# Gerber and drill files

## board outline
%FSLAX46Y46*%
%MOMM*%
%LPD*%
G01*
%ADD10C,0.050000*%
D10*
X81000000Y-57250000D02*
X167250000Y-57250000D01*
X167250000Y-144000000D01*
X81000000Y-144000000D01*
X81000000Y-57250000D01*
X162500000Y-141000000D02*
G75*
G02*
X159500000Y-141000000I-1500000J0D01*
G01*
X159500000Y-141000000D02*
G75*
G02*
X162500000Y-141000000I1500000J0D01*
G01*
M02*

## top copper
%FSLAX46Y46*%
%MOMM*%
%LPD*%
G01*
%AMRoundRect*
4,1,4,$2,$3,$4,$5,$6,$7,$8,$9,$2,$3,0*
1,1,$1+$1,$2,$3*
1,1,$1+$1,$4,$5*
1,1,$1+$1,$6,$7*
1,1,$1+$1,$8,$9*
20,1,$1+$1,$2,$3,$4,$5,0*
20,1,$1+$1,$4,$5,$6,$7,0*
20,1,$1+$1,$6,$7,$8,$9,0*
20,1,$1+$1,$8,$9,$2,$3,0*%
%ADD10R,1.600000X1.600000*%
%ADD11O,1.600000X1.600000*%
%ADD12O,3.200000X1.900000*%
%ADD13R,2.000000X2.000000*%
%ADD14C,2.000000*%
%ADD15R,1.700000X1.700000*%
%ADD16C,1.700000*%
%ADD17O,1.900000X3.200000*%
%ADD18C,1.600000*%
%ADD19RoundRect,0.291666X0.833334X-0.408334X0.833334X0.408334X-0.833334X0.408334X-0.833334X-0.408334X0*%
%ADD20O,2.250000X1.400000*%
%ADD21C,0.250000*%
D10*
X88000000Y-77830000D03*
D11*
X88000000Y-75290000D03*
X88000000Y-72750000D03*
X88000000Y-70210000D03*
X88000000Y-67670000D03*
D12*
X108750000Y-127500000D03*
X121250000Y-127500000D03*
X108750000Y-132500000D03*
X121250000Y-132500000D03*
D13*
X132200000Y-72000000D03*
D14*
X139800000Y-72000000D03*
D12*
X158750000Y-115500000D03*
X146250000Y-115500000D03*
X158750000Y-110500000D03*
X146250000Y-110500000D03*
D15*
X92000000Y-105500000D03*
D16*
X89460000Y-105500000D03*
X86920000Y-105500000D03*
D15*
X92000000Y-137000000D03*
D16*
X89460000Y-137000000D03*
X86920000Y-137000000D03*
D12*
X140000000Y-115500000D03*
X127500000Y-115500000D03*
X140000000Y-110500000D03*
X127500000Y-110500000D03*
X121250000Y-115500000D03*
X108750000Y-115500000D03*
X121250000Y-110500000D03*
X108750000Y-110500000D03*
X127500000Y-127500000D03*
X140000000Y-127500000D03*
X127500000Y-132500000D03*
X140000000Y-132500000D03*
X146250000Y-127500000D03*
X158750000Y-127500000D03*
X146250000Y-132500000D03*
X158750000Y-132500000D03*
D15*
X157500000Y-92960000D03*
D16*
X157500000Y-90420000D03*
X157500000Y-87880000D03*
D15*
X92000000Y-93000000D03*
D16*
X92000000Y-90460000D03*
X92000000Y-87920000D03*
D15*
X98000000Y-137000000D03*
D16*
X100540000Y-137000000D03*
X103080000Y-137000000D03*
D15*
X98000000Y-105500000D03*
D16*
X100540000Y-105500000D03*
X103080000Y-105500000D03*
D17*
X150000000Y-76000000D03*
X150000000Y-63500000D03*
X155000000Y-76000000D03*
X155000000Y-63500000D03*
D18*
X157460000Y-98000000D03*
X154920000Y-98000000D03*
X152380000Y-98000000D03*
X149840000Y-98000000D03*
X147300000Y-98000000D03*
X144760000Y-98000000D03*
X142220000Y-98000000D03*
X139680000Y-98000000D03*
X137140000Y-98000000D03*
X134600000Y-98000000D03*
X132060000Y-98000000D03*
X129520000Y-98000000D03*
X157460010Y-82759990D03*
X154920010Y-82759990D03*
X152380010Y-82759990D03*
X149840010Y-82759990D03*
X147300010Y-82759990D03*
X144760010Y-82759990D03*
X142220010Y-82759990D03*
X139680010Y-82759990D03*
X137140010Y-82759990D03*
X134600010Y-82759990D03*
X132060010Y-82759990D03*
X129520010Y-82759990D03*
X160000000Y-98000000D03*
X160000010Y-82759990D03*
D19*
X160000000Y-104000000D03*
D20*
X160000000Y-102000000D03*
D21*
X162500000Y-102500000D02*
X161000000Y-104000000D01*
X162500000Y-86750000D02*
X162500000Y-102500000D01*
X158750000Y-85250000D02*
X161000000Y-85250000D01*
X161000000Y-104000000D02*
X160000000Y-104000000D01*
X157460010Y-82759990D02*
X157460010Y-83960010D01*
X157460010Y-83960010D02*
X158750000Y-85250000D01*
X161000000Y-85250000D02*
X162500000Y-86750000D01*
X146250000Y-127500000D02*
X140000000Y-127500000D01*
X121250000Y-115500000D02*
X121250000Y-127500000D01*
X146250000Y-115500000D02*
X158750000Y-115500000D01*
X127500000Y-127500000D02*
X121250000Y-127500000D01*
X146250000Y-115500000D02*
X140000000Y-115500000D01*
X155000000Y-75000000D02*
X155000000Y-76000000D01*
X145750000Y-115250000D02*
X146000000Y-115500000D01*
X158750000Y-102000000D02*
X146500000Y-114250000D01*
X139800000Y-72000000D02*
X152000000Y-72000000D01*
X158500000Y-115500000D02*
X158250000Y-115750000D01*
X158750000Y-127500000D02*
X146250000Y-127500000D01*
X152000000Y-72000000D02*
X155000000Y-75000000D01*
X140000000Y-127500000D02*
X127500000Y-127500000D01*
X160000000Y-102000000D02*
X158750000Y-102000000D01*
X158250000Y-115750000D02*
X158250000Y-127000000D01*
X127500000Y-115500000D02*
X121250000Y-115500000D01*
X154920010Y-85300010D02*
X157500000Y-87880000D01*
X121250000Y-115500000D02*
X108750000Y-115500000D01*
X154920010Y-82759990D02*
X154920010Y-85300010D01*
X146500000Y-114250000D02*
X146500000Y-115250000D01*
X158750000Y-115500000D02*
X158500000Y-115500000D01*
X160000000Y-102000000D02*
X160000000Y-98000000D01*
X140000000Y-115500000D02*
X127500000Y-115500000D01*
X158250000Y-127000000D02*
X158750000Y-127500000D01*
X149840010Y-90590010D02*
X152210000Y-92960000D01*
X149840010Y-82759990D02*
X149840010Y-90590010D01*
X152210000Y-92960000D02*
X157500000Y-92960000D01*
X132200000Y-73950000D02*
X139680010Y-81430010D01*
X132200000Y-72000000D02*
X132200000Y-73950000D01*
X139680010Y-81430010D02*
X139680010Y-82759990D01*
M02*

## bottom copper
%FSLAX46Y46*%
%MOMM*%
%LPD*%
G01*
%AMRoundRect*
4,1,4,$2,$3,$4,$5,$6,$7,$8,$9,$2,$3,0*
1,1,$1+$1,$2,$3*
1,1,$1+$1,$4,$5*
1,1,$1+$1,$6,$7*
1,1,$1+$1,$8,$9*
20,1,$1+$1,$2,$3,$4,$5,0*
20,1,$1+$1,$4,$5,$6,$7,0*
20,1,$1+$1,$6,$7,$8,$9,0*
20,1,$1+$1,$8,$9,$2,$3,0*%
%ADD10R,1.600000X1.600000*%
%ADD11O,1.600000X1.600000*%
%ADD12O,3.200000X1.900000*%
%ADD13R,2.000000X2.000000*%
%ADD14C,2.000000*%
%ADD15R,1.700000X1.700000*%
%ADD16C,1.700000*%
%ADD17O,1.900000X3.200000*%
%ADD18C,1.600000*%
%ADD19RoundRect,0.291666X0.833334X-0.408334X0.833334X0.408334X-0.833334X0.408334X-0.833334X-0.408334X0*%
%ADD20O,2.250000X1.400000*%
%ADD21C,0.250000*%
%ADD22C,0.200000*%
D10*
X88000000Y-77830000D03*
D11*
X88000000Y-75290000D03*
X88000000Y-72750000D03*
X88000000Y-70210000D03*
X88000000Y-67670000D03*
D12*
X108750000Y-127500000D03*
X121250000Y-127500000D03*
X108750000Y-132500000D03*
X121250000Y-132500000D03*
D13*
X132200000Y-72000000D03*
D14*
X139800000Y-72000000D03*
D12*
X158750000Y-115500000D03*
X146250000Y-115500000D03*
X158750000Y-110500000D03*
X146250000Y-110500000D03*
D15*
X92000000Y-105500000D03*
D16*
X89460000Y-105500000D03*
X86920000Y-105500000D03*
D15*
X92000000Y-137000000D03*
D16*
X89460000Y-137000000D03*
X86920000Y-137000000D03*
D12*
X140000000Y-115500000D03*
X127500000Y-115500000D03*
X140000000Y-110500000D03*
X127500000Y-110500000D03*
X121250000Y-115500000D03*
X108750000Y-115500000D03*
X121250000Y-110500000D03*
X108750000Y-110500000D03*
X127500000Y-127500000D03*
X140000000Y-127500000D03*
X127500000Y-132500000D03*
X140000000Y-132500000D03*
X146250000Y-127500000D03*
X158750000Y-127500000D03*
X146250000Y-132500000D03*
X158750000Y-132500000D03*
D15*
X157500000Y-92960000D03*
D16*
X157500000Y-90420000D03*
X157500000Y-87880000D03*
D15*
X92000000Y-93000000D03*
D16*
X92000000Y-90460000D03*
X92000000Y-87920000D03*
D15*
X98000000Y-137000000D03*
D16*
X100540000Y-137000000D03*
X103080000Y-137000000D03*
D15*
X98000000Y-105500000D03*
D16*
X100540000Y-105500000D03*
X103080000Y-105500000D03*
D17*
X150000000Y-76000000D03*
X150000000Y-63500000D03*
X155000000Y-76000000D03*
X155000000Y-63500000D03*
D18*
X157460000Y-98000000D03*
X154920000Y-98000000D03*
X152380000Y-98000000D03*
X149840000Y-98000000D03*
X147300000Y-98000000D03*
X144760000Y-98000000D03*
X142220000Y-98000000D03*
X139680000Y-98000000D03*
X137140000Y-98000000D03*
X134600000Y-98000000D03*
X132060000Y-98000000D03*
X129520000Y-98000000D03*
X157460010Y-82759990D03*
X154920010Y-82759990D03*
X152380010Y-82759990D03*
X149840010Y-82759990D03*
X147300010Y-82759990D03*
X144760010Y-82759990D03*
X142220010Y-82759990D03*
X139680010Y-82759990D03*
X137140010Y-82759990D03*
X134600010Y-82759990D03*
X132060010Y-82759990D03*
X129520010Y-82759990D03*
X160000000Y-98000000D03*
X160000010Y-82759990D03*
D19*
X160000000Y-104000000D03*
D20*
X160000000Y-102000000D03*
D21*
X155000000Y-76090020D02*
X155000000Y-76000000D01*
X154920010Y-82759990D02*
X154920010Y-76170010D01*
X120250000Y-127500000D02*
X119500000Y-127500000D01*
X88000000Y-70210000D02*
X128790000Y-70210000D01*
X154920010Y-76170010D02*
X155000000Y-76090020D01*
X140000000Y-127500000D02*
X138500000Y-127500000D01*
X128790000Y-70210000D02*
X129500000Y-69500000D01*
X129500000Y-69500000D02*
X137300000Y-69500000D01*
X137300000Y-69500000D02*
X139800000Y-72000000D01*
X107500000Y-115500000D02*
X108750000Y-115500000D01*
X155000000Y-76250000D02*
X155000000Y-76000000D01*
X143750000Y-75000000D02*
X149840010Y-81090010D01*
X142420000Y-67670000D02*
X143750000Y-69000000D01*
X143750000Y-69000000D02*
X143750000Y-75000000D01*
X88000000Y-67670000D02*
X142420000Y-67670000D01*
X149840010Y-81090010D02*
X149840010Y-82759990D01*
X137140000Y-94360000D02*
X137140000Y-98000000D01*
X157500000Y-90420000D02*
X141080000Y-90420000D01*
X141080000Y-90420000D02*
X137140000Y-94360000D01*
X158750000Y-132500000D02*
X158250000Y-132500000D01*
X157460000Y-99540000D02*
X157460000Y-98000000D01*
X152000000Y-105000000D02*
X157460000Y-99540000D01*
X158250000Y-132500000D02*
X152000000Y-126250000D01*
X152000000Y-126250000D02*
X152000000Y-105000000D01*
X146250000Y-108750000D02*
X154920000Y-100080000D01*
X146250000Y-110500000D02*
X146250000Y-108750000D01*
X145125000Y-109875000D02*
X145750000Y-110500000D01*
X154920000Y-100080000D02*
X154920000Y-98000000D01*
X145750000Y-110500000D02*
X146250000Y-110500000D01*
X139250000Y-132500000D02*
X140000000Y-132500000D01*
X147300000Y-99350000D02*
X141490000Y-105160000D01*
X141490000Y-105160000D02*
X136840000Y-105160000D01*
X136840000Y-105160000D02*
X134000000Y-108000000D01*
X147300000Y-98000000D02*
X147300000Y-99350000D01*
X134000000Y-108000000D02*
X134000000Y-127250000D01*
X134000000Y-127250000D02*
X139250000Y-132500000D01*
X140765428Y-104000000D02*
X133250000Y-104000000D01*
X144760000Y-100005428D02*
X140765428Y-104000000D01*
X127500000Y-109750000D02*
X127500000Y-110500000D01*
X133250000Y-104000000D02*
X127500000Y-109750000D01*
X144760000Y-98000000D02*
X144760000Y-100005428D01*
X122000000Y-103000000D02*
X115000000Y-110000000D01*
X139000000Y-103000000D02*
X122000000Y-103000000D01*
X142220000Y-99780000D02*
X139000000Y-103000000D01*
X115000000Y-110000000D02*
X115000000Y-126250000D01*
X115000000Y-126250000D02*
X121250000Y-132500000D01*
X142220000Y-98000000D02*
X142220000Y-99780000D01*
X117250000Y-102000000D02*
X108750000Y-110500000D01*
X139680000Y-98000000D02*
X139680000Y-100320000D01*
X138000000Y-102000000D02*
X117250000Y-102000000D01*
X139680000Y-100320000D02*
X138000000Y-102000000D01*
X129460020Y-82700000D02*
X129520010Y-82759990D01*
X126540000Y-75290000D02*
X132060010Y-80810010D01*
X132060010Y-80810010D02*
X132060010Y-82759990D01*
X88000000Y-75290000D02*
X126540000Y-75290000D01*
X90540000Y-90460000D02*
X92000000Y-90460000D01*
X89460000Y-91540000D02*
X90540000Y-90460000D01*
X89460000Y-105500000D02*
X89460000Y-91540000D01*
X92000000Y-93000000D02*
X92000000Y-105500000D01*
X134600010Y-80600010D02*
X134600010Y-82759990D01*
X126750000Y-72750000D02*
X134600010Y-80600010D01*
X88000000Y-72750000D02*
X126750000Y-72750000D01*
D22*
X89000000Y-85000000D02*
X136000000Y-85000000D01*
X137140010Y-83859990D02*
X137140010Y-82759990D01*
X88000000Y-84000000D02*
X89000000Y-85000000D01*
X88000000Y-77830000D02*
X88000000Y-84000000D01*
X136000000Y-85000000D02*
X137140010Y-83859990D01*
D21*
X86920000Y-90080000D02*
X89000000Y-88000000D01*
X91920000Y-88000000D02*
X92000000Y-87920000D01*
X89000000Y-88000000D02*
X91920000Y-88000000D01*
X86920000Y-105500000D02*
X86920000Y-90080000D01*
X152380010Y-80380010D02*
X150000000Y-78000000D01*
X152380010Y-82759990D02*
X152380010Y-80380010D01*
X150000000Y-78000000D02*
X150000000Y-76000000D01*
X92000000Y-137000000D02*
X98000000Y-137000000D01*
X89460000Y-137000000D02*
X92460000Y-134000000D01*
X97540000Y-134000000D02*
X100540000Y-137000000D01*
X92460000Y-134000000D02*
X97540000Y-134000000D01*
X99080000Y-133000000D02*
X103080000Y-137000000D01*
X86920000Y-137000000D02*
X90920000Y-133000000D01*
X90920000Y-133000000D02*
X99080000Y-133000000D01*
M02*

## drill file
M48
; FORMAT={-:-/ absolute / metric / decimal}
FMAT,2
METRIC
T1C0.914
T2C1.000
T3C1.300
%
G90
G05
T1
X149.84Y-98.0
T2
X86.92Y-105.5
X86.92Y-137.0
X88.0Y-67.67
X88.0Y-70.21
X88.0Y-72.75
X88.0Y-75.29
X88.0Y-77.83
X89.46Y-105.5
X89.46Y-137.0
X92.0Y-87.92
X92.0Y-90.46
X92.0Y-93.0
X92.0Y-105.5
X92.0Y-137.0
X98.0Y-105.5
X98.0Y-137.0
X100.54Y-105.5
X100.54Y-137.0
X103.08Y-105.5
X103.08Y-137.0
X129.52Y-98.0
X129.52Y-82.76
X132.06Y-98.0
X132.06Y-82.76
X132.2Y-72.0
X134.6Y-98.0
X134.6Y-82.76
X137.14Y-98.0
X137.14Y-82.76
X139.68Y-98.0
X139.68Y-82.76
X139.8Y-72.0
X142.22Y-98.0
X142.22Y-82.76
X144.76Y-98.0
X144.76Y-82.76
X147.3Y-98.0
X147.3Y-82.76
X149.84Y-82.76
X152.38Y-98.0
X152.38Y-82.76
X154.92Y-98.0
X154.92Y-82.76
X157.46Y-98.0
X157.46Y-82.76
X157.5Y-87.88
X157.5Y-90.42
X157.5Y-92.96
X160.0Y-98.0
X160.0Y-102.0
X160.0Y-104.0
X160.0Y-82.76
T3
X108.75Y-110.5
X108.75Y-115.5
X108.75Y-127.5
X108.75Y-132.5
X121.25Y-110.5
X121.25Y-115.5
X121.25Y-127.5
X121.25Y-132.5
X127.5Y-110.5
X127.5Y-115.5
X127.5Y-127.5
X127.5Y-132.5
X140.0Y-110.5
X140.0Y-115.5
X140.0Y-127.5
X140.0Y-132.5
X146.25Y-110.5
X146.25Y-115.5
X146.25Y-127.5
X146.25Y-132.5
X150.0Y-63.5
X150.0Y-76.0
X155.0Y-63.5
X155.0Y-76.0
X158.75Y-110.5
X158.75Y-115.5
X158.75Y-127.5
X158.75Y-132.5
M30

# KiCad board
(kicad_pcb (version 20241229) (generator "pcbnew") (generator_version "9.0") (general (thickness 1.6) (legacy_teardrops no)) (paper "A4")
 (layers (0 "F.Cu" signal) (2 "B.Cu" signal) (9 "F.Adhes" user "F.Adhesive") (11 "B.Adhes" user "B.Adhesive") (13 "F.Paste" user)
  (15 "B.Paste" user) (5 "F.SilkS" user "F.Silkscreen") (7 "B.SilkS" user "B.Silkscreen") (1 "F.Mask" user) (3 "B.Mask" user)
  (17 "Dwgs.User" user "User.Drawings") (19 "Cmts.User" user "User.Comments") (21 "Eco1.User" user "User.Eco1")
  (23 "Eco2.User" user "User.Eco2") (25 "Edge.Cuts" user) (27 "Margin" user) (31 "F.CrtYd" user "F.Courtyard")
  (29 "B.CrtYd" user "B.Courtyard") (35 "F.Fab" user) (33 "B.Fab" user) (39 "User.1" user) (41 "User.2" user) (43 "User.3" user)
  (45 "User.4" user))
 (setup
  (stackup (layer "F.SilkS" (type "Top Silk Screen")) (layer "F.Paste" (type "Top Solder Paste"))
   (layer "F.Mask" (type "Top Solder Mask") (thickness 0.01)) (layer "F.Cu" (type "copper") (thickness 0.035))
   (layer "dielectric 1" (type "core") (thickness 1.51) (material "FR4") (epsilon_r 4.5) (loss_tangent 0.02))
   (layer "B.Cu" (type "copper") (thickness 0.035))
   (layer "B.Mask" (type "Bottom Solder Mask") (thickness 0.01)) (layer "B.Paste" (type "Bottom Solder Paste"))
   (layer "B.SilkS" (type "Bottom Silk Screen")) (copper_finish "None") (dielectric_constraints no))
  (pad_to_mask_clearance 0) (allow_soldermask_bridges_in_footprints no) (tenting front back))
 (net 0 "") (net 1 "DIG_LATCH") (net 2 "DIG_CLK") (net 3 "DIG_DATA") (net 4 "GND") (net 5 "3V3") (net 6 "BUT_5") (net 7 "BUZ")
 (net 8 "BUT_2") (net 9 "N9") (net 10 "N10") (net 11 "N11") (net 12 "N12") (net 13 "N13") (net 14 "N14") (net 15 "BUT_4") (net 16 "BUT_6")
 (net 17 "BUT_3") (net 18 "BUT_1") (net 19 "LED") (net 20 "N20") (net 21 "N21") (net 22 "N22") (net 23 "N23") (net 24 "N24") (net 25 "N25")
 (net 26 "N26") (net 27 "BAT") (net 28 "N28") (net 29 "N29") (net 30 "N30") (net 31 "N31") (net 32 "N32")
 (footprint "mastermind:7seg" (layer "F.Cu") (at 94.5 69.25)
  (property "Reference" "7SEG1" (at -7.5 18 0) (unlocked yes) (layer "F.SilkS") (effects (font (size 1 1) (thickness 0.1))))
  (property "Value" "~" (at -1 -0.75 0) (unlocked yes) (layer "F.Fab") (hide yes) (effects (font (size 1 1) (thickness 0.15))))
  (pad "1" thru_hole rect (at -6.5 8.58 180) (size 1.6 1.6) (drill 1) (layers "*.Cu" "*.Mask") (remove_unused_layers no) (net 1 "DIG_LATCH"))
  (pad "2" thru_hole oval (at -6.5 6.04 180) (size 1.6 1.6) (drill 1) (layers "*.Cu" "*.Mask") (remove_unused_layers no) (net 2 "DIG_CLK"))
  (pad "3" thru_hole oval (at -6.5 3.5 180) (size 1.6 1.6) (drill 1) (layers "*.Cu" "*.Mask") (remove_unused_layers no) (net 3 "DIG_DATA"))
  (pad "4" thru_hole oval (at -6.5 0.96 180) (size 1.6 1.6) (drill 1) (layers "*.Cu" "*.Mask") (remove_unused_layers no) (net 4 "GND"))
  (pad "5" thru_hole oval (at -6.5 -1.58 180) (size 1.6 1.6) (drill 1) (layers "*.Cu" "*.Mask") (remove_unused_layers no) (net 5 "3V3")))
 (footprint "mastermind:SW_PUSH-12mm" (layer "F.Cu") (at 108.75 127.5)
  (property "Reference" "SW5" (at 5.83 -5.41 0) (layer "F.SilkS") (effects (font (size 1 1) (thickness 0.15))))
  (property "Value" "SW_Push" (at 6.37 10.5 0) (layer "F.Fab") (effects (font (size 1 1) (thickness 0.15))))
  (pad "1" thru_hole oval (at 0 0) (size 3.2 1.9) (drill 1.3) (layers "*.Cu" "*.Mask") (remove_unused_layers no) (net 4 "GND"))
  (pad "1" thru_hole oval (at 12.5 0) (size 3.2 1.9) (drill 1.3) (layers "*.Cu" "*.Mask") (remove_unused_layers no) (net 4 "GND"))
  (pad "2" thru_hole oval (at 0 5) (size 3.2 1.9) (drill 1.3) (layers "*.Cu" "*.Mask") (remove_unused_layers no) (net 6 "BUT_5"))
  (pad "2" thru_hole oval (at 12.5 5) (size 3.2 1.9) (drill 1.3) (layers "*.Cu" "*.Mask") (remove_unused_layers no) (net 6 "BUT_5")))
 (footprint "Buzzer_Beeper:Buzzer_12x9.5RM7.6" (layer "F.Cu") (at 132.2 72)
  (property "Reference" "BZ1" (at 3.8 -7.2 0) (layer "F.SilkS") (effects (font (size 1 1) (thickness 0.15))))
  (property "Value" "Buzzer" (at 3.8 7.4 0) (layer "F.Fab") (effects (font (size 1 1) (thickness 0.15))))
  (pad "1" thru_hole rect (at 0 0) (size 2 2) (drill 1) (layers "*.Cu" "*.Mask") (remove_unused_layers no) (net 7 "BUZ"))
  (pad "2" thru_hole circle (at 7.6 0) (size 2 2) (drill 1) (layers "*.Cu" "*.Mask") (remove_unused_layers no) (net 4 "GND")))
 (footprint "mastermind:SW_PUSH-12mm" (layer "F.Cu") (at 158.75 115.5 180)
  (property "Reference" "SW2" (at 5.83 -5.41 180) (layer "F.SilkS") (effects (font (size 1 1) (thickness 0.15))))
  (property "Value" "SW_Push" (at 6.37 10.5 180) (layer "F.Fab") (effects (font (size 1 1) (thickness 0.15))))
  (pad "1" thru_hole oval (at 0 0 180) (size 3.2 1.9) (drill 1.3) (layers "*.Cu" "*.Mask") (remove_unused_layers no) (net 4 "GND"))
  (pad "1" thru_hole oval (at 12.5 0 180) (size 3.2 1.9) (drill 1.3) (layers "*.Cu" "*.Mask") (remove_unused_layers no) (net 4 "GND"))
  (pad "2" thru_hole oval (at 0 5 180) (size 3.2 1.9) (drill 1.3) (layers "*.Cu" "*.Mask") (remove_unused_layers no) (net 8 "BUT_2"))
  (pad "2" thru_hole oval (at 12.5 5 180) (size 3.2 1.9) (drill 1.3) (layers "*.Cu" "*.Mask") (remove_unused_layers no) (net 8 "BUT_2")))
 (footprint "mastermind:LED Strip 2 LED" (layer "F.Cu") (at 89.75 129.75 -90)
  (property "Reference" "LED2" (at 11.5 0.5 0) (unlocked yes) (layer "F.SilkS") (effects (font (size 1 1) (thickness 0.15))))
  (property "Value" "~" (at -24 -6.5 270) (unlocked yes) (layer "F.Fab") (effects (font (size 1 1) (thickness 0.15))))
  (pad "1" thru_hole rect (at -24.25 -2.25 270) (size 1.7 1.7) (drill 1) (layers "*.Cu" "*.Mask") (remove_unused_layers no) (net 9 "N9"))
  (pad "2" thru_hole circle (at -24.25 0.29 270) (size 1.7 1.7) (drill 1) (layers "*.Cu" "*.Mask") (remove_unused_layers no) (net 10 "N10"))
  (pad "3" thru_hole circle (at -24.25 2.83 270) (size 1.7 1.7) (drill 1) (layers "*.Cu" "*.Mask") (remove_unused_layers no) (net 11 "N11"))
  (pad "4" thru_hole rect (at 7.25 -2.25 270) (size 1.7 1.7) (drill 1) (layers "*.Cu" "*.Mask") (remove_unused_layers no) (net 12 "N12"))
  (pad "5" thru_hole circle (at 7.25 0.29 270) (size 1.7 1.7) (drill 1) (layers "*.Cu" "*.Mask") (remove_unused_layers no) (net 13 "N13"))
  (pad "6" thru_hole circle (at 7.25 2.83 270) (size 1.7 1.7) (drill 1) (layers "*.Cu" "*.Mask") (remove_unused_layers no) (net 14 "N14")))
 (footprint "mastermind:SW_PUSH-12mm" (layer "F.Cu") (at 140 115.5 180)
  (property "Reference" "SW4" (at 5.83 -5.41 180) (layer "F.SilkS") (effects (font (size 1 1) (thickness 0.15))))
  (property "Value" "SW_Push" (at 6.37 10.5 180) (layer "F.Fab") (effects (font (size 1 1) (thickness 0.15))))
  (pad "1" thru_hole oval (at 0 0 180) (size 3.2 1.9) (drill 1.3) (layers "*.Cu" "*.Mask") (remove_unused_layers no) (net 4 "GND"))
  (pad "1" thru_hole oval (at 12.5 0 180) (size 3.2 1.9) (drill 1.3) (layers "*.Cu" "*.Mask") (remove_unused_layers no) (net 4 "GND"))
  (pad "2" thru_hole oval (at 0 5 180) (size 3.2 1.9) (drill 1.3) (layers "*.Cu" "*.Mask") (remove_unused_layers no) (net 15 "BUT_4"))
  (pad "2" thru_hole oval (at 12.5 5 180) (size 3.2 1.9) (drill 1.3) (layers "*.Cu" "*.Mask") (remove_unused_layers no) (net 15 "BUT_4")))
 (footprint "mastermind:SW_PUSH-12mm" (layer "F.Cu") (at 121.25 115.5 180)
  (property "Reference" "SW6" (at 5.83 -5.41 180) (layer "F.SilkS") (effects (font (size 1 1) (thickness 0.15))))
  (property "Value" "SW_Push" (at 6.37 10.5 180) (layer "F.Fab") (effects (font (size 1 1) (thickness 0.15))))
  (pad "1" thru_hole oval (at 0 0 180) (size 3.2 1.9) (drill 1.3) (layers "*.Cu" "*.Mask") (remove_unused_layers no) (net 4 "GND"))
  (pad "1" thru_hole oval (at 12.5 0 180) (size 3.2 1.9) (drill 1.3) (layers "*.Cu" "*.Mask") (remove_unused_layers no) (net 4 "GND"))
  (pad "2" thru_hole oval (at 0 5 180) (size 3.2 1.9) (drill 1.3) (layers "*.Cu" "*.Mask") (remove_unused_layers no) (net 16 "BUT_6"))
  (pad "2" thru_hole oval (at 12.5 5 180) (size 3.2 1.9) (drill 1.3) (layers "*.Cu" "*.Mask") (remove_unused_layers no) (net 16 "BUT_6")))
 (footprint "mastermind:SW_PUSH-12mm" (layer "F.Cu") (at 127.5 127.5)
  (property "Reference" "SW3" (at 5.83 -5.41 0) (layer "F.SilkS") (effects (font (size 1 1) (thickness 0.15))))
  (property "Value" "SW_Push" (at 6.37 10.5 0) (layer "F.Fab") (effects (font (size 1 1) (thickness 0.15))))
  (pad "1" thru_hole oval (at 0 0) (size 3.2 1.9) (drill 1.3) (layers "*.Cu" "*.Mask") (remove_unused_layers no) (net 4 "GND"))
  (pad "1" thru_hole oval (at 12.5 0) (size 3.2 1.9) (drill 1.3) (layers "*.Cu" "*.Mask") (remove_unused_layers no) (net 4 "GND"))
  (pad "2" thru_hole oval (at 0 5) (size 3.2 1.9) (drill 1.3) (layers "*.Cu" "*.Mask") (remove_unused_layers no) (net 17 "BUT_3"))
  (pad "2" thru_hole oval (at 12.5 5) (size 3.2 1.9) (drill 1.3) (layers "*.Cu" "*.Mask") (remove_unused_layers no) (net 17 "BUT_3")))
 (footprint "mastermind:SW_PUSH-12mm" (layer "F.Cu") (at 146.25 127.5)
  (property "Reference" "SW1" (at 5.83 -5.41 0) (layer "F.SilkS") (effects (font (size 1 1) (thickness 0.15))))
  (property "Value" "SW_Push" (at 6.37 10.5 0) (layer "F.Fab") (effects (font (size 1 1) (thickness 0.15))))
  (pad "1" thru_hole oval (at 0 0) (size 3.2 1.9) (drill 1.3) (layers "*.Cu" "*.Mask") (remove_unused_layers no) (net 4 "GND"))
  (pad "1" thru_hole oval (at 12.5 0) (size 3.2 1.9) (drill 1.3) (layers "*.Cu" "*.Mask") (remove_unused_layers no) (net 4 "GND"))
  (pad "2" thru_hole oval (at 0 5) (size 3.2 1.9) (drill 1.3) (layers "*.Cu" "*.Mask") (remove_unused_layers no) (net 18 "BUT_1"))
  (pad "2" thru_hole oval (at 12.5 5) (size 3.2 1.9) (drill 1.3) (layers "*.Cu" "*.Mask") (remove_unused_layers no) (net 18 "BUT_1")))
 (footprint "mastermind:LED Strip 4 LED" (layer "F.Cu") (at 133.25 90.71 180)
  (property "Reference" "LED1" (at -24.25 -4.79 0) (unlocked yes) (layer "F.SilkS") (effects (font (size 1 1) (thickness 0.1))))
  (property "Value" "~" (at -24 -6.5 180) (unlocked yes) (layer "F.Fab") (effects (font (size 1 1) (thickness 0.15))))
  (pad "1" thru_hole rect (at -24.25 -2.25 180) (size 1.7 1.7) (drill 1) (layers "*.Cu" "*.Mask") (remove_unused_layers no) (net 5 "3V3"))
  (pad "2" thru_hole circle (at -24.25 0.29 180) (size 1.7 1.7) (drill 1) (layers "*.Cu" "*.Mask") (remove_unused_layers no) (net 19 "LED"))
  (pad "3" thru_hole circle (at -24.25 2.83 180) (size 1.7 1.7) (drill 1) (layers "*.Cu" "*.Mask") (remove_unused_layers no) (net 4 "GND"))
  (pad "4" thru_hole rect (at 41.25 -2.29 180) (size 1.7 1.7) (drill 1) (layers "*.Cu" "*.Mask") (remove_unused_layers no) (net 9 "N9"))
  (pad "5" thru_hole circle (at 41.25 0.25 180) (size 1.7 1.7) (drill 1) (layers "*.Cu" "*.Mask") (remove_unused_layers no) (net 10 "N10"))
  (pad "6" thru_hole circle (at 41.25 2.79 180) (size 1.7 1.7) (drill 1) (layers "*.Cu" "*.Mask") (remove_unused_layers no) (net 11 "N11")))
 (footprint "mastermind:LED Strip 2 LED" (layer "F.Cu") (at 100.25 112.75 90)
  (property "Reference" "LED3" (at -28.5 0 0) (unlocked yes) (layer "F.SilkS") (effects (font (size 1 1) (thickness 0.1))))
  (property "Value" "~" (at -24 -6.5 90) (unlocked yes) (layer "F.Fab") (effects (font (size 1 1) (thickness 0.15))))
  (pad "1" thru_hole rect (at -24.25 -2.25 90) (size 1.7 1.7) (drill 1) (layers "*.Cu" "*.Mask") (remove_unused_layers no) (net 12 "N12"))
  (pad "2" thru_hole circle (at -24.25 0.29 90) (size 1.7 1.7) (drill 1) (layers "*.Cu" "*.Mask") (remove_unused_layers no) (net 13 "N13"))
  (pad "3" thru_hole circle (at -24.25 2.83 90) (size 1.7 1.7) (drill 1) (layers "*.Cu" "*.Mask") (remove_unused_layers no) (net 14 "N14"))
  (pad "4" thru_hole rect (at 7.25 -2.25 90) (size 1.7 1.7) (drill 1) (layers "*.Cu" "*.Mask") (remove_unused_layers no) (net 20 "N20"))
  (pad "5" thru_hole circle (at 7.25 0.29 90) (size 1.7 1.7) (drill 1) (layers "*.Cu" "*.Mask") (remove_unused_layers no) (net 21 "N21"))
  (pad "6" thru_hole circle (at 7.25 2.83 90) (size 1.7 1.7) (drill 1) (layers "*.Cu" "*.Mask") (remove_unused_layers no) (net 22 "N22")))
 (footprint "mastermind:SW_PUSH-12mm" (layer "F.Cu") (at 150 76 90)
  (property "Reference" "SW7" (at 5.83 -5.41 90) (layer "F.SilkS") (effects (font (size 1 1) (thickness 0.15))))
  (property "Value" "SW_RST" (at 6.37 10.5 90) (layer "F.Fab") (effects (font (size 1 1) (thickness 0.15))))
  (pad "1" thru_hole oval (at 0 0 90) (size 3.2 1.9) (drill 1.3) (layers "*.Cu" "*.Mask") (remove_unused_layers no) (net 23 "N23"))
  (pad "1" thru_hole oval (at 12.5 0 90) (size 3.2 1.9) (drill 1.3) (layers "*.Cu" "*.Mask") (remove_unused_layers no) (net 23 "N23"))
  (pad "2" thru_hole oval (at 0 5 90) (size 3.2 1.9) (drill 1.3) (layers "*.Cu" "*.Mask") (remove_unused_layers no) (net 4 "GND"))
  (pad "2" thru_hole oval (at 12.5 5 90) (size 3.2 1.9) (drill 1.3) (layers "*.Cu" "*.Mask") (remove_unused_layers no) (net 4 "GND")))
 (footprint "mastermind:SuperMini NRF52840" (layer "B.Cu") (at 160 98 90)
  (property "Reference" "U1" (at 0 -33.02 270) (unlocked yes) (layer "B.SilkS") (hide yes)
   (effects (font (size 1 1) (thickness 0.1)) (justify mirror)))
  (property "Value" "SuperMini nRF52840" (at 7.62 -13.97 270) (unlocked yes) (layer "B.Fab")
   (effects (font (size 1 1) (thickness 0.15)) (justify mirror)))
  (pad "1" thru_hole circle (at 0 -2.54 180) (size 1.6 1.6) (drill 1) (layers "*.Cu" "*.Mask") (remove_unused_layers no) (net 18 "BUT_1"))
  (pad "2" thru_hole circle (at 0 -5.08 180) (size 1.6 1.6) (drill 1) (layers "*.Cu" "*.Mask") (remove_unused_layers no) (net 8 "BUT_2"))
  (pad "3" thru_hole circle (at 0 -7.62 180) (size 1.6 1.6) (drill 1) (layers "*.Cu" "*.Mask") (remove_unused_layers no) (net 4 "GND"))
  (pad "4" thru_hole circle (at 0 -10.16) (size 1.6 1.6) (drill 0.9144) (layers "*.Cu" "*.Mask") (remove_unused_layers no) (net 4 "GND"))
  (pad "5" thru_hole circle (at 0 -12.7 180) (size 1.6 1.6) (drill 1) (layers "*.Cu" "*.Mask") (remove_unused_layers no) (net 17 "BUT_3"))
  (pad "6" thru_hole circle (at 0 -15.24 180) (size 1.6 1.6) (drill 1) (layers "*.Cu" "*.Mask") (remove_unused_layers no) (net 15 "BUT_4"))
  (pad "7" thru_hole circle (at 0 -17.78 180) (size 1.6 1.6) (drill 1) (layers "*.Cu" "*.Mask") (remove_unused_layers no) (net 6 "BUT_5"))
  (pad "8" thru_hole circle (at 0 -20.32 180) (size 1.6 1.6) (drill 1) (layers "*.Cu" "*.Mask") (remove_unused_layers no) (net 16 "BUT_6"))
  (pad "9" thru_hole circle (at 0 -22.86 180) (size 1.6 1.6) (drill 1) (layers "*.Cu" "*.Mask") (remove_unused_layers no) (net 19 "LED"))
  (pad "10" thru_hole circle (at 0 -25.4 180) (size 1.6 1.6) (drill 1) (layers "*.Cu" "*.Mask") (remove_unused_layers no) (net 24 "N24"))
  (pad "11" thru_hole circle (at 0 -27.94 180) (size 1.6 1.6) (drill 1) (layers "*.Cu" "*.Mask") (remove_unused_layers no) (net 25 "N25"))
  (pad "12" thru_hole circle (at 0 -30.48 180) (size 1.6 1.6) (drill 1) (layers "*.Cu" "*.Mask") (remove_unused_layers no) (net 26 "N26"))
  (pad "13" thru_hole circle (at 15.24001 -2.53999) (size 1.6 1.6) (drill 1) (layers "*.Cu" "*.Mask") (remove_unused_layers no)
   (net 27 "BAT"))
  (pad "14" thru_hole circle (at 15.24001 -5.07999) (size 1.6 1.6) (drill 1) (layers "*.Cu" "*.Mask") (remove_unused_layers no)
   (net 4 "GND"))
  (pad "15" thru_hole circle (at 15.24001 -7.61999) (size 1.6 1.6) (drill 1) (layers "*.Cu" "*.Mask") (remove_unused_layers no)
   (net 23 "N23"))
  (pad "16" thru_hole circle (at 15.24001 -10.15999) (size 1.6 1.6) (drill 1) (layers "*.Cu" "*.Mask") (remove_unused_layers no)
   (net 5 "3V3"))
  (pad "17" thru_hole circle (at 15.24001 -12.69999) (size 1.6 1.6) (drill 1) (layers "*.Cu" "*.Mask") (remove_unused_layers no)
   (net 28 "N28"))
  (pad "18" thru_hole circle (at 15.24001 -15.23999) (size 1.6 1.6) (drill 1) (layers "*.Cu" "*.Mask") (remove_unused_layers no)
   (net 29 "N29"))
  (pad "19" thru_hole circle (at 15.24001 -17.77999) (size 1.6 1.6) (drill 1) (layers "*.Cu" "*.Mask") (remove_unused_layers no)
   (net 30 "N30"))
  (pad "20" thru_hole circle (at 15.24001 -20.31999) (size 1.6 1.6) (drill 1) (layers "*.Cu" "*.Mask") (remove_unused_layers no)
   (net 7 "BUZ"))
  (pad "21" thru_hole circle (at 15.24001 -22.85999) (size 1.6 1.6) (drill 1) (layers "*.Cu" "*.Mask") (remove_unused_layers no)
   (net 1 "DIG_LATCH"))
  (pad "22" thru_hole circle (at 15.24001 -25.39999) (size 1.6 1.6) (drill 1) (layers "*.Cu" "*.Mask") (remove_unused_layers no)
   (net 3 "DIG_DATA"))
  (pad "23" thru_hole circle (at 15.24001 -27.93999) (size 1.6 1.6) (drill 1) (layers "*.Cu" "*.Mask") (remove_unused_layers no)
   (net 2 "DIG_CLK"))
  (pad "24" thru_hole circle (at 15.24001 -30.47999 180) (size 1.6 1.6) (drill 1) (layers "*.Cu" "*.Mask") (remove_unused_layers no)
   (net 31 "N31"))
  (pad "28" thru_hole circle (at 0 0 180) (size 1.6 1.6) (drill 1) (layers "*.Cu" "*.Mask") (remove_unused_layers no) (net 4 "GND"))
  (pad "29" thru_hole circle (at 15.24001 0.00001) (size 1.6 1.6) (drill 1) (layers "*.Cu" "*.Mask") (remove_unused_layers no)
   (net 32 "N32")))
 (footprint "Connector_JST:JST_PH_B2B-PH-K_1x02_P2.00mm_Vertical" (layer "B.Cu") (at 160 104 90)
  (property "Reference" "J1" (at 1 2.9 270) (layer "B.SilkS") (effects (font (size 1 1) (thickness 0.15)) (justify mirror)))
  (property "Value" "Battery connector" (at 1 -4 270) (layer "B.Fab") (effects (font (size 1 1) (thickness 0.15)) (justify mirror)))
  (pad "1" thru_hole roundrect (at 0 0 90) (size 1.4 2.25) (drill 1) (layers "*.Cu" "*.Mask") (remove_unused_layers no)
   (roundrect_rratio 0.208333) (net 27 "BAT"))
  (pad "2" thru_hole oval (at 2 0 90) (size 1.4 2.25) (drill 1) (layers "*.Cu" "*.Mask") (remove_unused_layers no) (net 4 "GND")))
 (gr_rect (start 81 57.25) (end 167.25 144) (stroke (width 0.05) (type default)) (fill no) (layer "Edge.Cuts"))
 (gr_circle (center 161 141) (end 162.5 141) (stroke (width 0.05) (type solid)) (fill no) (layer "Edge.Cuts"))
 (segment (start 162.5 102.5) (end 161 104) (width 0.25) (layer "F.Cu") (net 27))
 (segment (start 162.5 86.75) (end 162.5 102.5) (width 0.25) (layer "F.Cu") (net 27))
 (segment (start 158.75 85.25) (end 161 85.25) (width 0.25) (layer "F.Cu") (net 27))
 (segment (start 161 104) (end 160 104) (width 0.25) (layer "F.Cu") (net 27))
 (segment (start 157.46001 82.75999) (end 157.46001 83.96001) (width 0.25) (layer "F.Cu") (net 27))
 (segment (start 157.46001 83.96001) (end 158.75 85.25) (width 0.25) (layer "F.Cu") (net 27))
 (segment (start 161 85.25) (end 162.5 86.75) (width 0.25) (layer "F.Cu") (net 27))
 (segment (start 146.25 127.5) (end 140 127.5) (width 0.25) (layer "F.Cu") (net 4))
 (segment (start 121.25 115.5) (end 121.25 127.5) (width 0.25) (layer "F.Cu") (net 4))
 (segment (start 146.25 115.5) (end 158.75 115.5) (width 0.25) (layer "F.Cu") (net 4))
 (segment (start 127.5 127.5) (end 121.25 127.5) (width 0.25) (layer "F.Cu") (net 4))
 (segment (start 146.25 115.5) (end 140 115.5) (width 0.25) (layer "F.Cu") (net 4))
 (segment (start 155 75) (end 155 76) (width 0.25) (layer "F.Cu") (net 4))
 (segment (start 145.75 115.25) (end 146 115.5) (width 0.25) (layer "F.Cu") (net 4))
 (segment (start 158.75 102) (end 146.5 114.25) (width 0.25) (layer "F.Cu") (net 4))
 (segment (start 139.8 72) (end 152 72) (width 0.25) (layer "F.Cu") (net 4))
 (segment (start 158.5 115.5) (end 158.25 115.75) (width 0.25) (layer "F.Cu") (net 4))
 (segment (start 158.75 127.5) (end 146.25 127.5) (width 0.25) (layer "F.Cu") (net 4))
 (segment (start 152 72) (end 155 75) (width 0.25) (layer "F.Cu") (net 4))
 (segment (start 140 127.5) (end 127.5 127.5) (width 0.25) (layer "F.Cu") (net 4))
 (segment (start 160 102) (end 158.75 102) (width 0.25) (layer "F.Cu") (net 4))
 (segment (start 158.25 115.75) (end 158.25 127) (width 0.25) (layer "F.Cu") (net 4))
 (segment (start 127.5 115.5) (end 121.25 115.5) (width 0.25) (layer "F.Cu") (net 4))
 (segment (start 154.92001 85.30001) (end 157.5 87.88) (width 0.25) (layer "F.Cu") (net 4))
 (segment (start 121.25 115.5) (end 108.75 115.5) (width 0.25) (layer "F.Cu") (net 4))
 (segment (start 154.92001 82.75999) (end 154.92001 85.30001) (width 0.25) (layer "F.Cu") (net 4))
 (segment (start 146.5 114.25) (end 146.5 115.25) (width 0.25) (layer "F.Cu") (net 4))
 (segment (start 158.75 115.5) (end 158.5 115.5) (width 0.25) (layer "F.Cu") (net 4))
 (segment (start 160 102) (end 160 98) (width 0.25) (layer "F.Cu") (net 4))
 (segment (start 140 115.5) (end 127.5 115.5) (width 0.25) (layer "F.Cu") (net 4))
 (segment (start 158.25 127) (end 158.75 127.5) (width 0.25) (layer "F.Cu") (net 4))
 (segment (start 155 76.09002) (end 155 76) (width 0.25) (layer "B.Cu") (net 4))
 (segment (start 154.92001 82.75999) (end 154.92001 76.17001) (width 0.25) (layer "B.Cu") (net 4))
 (segment (start 120.25 127.5) (end 119.5 127.5) (width 0.25) (layer "B.Cu") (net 4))
 (segment (start 88 70.21) (end 128.79 70.21) (width 0.25) (layer "B.Cu") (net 4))
 (segment (start 154.92001 76.17001) (end 155 76.09002) (width 0.25) (layer "B.Cu") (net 4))
 (segment (start 140 127.5) (end 138.5 127.5) (width 0.25) (layer "B.Cu") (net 4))
 (segment (start 128.79 70.21) (end 129.5 69.5) (width 0.25) (layer "B.Cu") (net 4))
 (segment (start 129.5 69.5) (end 137.3 69.5) (width 0.25) (layer "B.Cu") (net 4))
 (segment (start 137.3 69.5) (end 139.8 72) (width 0.25) (layer "B.Cu") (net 4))
 (segment (start 107.5 115.5) (end 108.75 115.5) (width 0.25) (layer "B.Cu") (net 4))
 (segment (start 155 76.25) (end 155 76) (width 0.25) (layer "B.Cu") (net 4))
 (segment (start 149.84001 90.59001) (end 152.21 92.96) (width 0.25) (layer "F.Cu") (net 5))
 (segment (start 149.84001 82.75999) (end 149.84001 90.59001) (width 0.25) (layer "F.Cu") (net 5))
 (segment (start 152.21 92.96) (end 157.5 92.96) (width 0.25) (layer "F.Cu") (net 5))
 (segment (start 143.75 75) (end 149.84001 81.09001) (width 0.25) (layer "B.Cu") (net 5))
 (segment (start 142.42 67.67) (end 143.75 69) (width 0.25) (layer "B.Cu") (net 5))
 (segment (start 143.75 69) (end 143.75 75) (width 0.25) (layer "B.Cu") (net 5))
 (segment (start 88 67.67) (end 142.42 67.67) (width 0.25) (layer "B.Cu") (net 5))
 (segment (start 149.84001 81.09001) (end 149.84001 82.75999) (width 0.25) (layer "B.Cu") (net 5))
 (segment (start 137.14 94.36) (end 137.14 98) (width 0.25) (layer "B.Cu") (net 19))
 (segment (start 157.5 90.42) (end 141.08 90.42) (width 0.25) (layer "B.Cu") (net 19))
 (segment (start 141.08 90.42) (end 137.14 94.36) (width 0.25) (layer "B.Cu") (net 19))
 (segment (start 158.75 132.5) (end 158.25 132.5) (width 0.25) (layer "B.Cu") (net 18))
 (segment (start 157.46 99.54) (end 157.46 98) (width 0.25) (layer "B.Cu") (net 18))
 (segment (start 152 105) (end 157.46 99.54) (width 0.25) (layer "B.Cu") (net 18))
 (segment (start 158.25 132.5) (end 152 126.25) (width 0.25) (layer "B.Cu") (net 18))
 (segment (start 152 126.25) (end 152 105) (width 0.25) (layer "B.Cu") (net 18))
 (segment (start 146.25 108.75) (end 154.92 100.08) (width 0.25) (layer "B.Cu") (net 8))
 (segment (start 146.25 110.5) (end 146.25 108.75) (width 0.25) (layer "B.Cu") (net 8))
 (segment (start 145.125 109.875) (end 145.75 110.5) (width 0.25) (layer "B.Cu") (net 8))
 (segment (start 154.92 100.08) (end 154.92 98) (width 0.25) (layer "B.Cu") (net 8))
 (segment (start 145.75 110.5) (end 146.25 110.5) (width 0.25) (layer "B.Cu") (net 8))
 (segment (start 139.25 132.5) (end 140 132.5) (width 0.25) (layer "B.Cu") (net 17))
 (segment (start 147.3 99.35) (end 141.49 105.16) (width 0.25) (layer "B.Cu") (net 17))
 (segment (start 141.49 105.16) (end 136.84 105.16) (width 0.25) (layer "B.Cu") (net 17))
 (segment (start 136.84 105.16) (end 134 108) (width 0.25) (layer "B.Cu") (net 17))
 (segment (start 147.3 98) (end 147.3 99.35) (width 0.25) (layer "B.Cu") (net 17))
 (segment (start 134 108) (end 134 127.25) (width 0.25) (layer "B.Cu") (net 17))
 (segment (start 134 127.25) (end 139.25 132.5) (width 0.25) (layer "B.Cu") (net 17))
 (segment (start 140.765428 104) (end 133.25 104) (width 0.25) (layer "B.Cu") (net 15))
 (segment (start 144.76 100.005428) (end 140.765428 104) (width 0.25) (layer "B.Cu") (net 15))
 (segment (start 127.5 109.75) (end 127.5 110.5) (width 0.25) (layer "B.Cu") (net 15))
 (segment (start 133.25 104) (end 127.5 109.75) (width 0.25) (layer "B.Cu") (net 15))
 (segment (start 144.76 98) (end 144.76 100.005428) (width 0.25) (layer "B.Cu") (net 15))
 (segment (start 122 103) (end 115 110) (width 0.25) (layer "B.Cu") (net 6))
 (segment (start 139 103) (end 122 103) (width 0.25) (layer "B.Cu") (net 6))
 (segment (start 142.22 99.78) (end 139 103) (width 0.25) (layer "B.Cu") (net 6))
 (segment (start 115 110) (end 115 126.25) (width 0.25) (layer "B.Cu") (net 6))
 (segment (start 115 126.25) (end 121.25 132.5) (width 0.25) (layer "B.Cu") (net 6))
 (segment (start 142.22 98) (end 142.22 99.78) (width 0.25) (layer "B.Cu") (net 6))
 (segment (start 117.25 102) (end 108.75 110.5) (width 0.25) (layer "B.Cu") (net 16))
 (segment (start 139.68 98) (end 139.68 100.32) (width 0.25) (layer "B.Cu") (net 16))
 (segment (start 138 102) (end 117.25 102) (width 0.25) (layer "B.Cu") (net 16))
 (segment (start 139.68 100.32) (end 138 102) (width 0.25) (layer "B.Cu") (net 16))
 (segment (start 129.46002 82.7) (end 129.52001 82.75999) (width 0.25) (layer "B.Cu") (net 31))
 (segment (start 132.2 73.95) (end 139.68001 81.43001) (width 0.25) (layer "F.Cu") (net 7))
 (segment (start 132.2 72) (end 132.2 73.95) (width 0.25) (layer "F.Cu") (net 7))
 (segment (start 139.68001 81.43001) (end 139.68001 82.75999) (width 0.25) (layer "F.Cu") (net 7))
 (segment (start 126.54 75.29) (end 132.06001 80.81001) (width 0.25) (layer "B.Cu") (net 2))
 (segment (start 132.06001 80.81001) (end 132.06001 82.75999) (width 0.25) (layer "B.Cu") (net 2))
 (segment (start 88 75.29) (end 126.54 75.29) (width 0.25) (layer "B.Cu") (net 2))
 (segment (start 90.54 90.46) (end 92 90.46) (width 0.25) (layer "B.Cu") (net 10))
 (segment (start 89.46 91.54) (end 90.54 90.46) (width 0.25) (layer "B.Cu") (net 10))
 (segment (start 89.46 105.5) (end 89.46 91.54) (width 0.25) (layer "B.Cu") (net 10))
 (segment (start 92 93) (end 92 105.5) (width 0.25) (layer "B.Cu") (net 9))
 (segment (start 134.60001 80.60001) (end 134.60001 82.75999) (width 0.25) (layer "B.Cu") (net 3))
 (segment (start 126.75 72.75) (end 134.60001 80.60001) (width 0.25) (layer "B.Cu") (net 3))
 (segment (start 88 72.75) (end 126.75 72.75) (width 0.25) (layer "B.Cu") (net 3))
 (segment (start 89 85) (end 136 85) (width 0.2) (layer "B.Cu") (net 1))
 (segment (start 137.14001 83.85999) (end 137.14001 82.75999) (width 0.2) (layer "B.Cu") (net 1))
 (segment (start 88 84) (end 89 85) (width 0.2) (layer "B.Cu") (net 1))
 (segment (start 88 77.83) (end 88 84) (width 0.2) (layer "B.Cu") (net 1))
 (segment (start 136 85) (end 137.14001 83.85999) (width 0.2) (layer "B.Cu") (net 1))
 (segment (start 86.92 90.08) (end 89 88) (width 0.25) (layer "B.Cu") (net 11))
 (segment (start 91.92 88) (end 92 87.92) (width 0.25) (layer "B.Cu") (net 11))
 (segment (start 89 88) (end 91.92 88) (width 0.25) (layer "B.Cu") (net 11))
 (segment (start 86.92 105.5) (end 86.92 90.08) (width 0.25) (layer "B.Cu") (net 11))
 (segment (start 152.38001 80.38001) (end 150 78) (width 0.25) (layer "B.Cu") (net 23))
 (segment (start 152.38001 82.75999) (end 152.38001 80.38001) (width 0.25) (layer "B.Cu") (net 23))
 (segment (start 150 78) (end 150 76) (width 0.25) (layer "B.Cu") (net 23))
 (segment (start 92 137) (end 98 137) (width 0.25) (layer "B.Cu") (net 12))
 (segment (start 89.46 137) (end 92.46 134) (width 0.25) (layer "B.Cu") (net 13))
 (segment (start 97.54 134) (end 100.54 137) (width 0.25) (layer "B.Cu") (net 13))
 (segment (start 92.46 134) (end 97.54 134) (width 0.25) (layer "B.Cu") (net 13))
 (segment (start 99.08 133) (end 103.08 137) (width 0.25) (layer "B.Cu") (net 14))
 (segment (start 86.92 137) (end 90.92 133) (width 0.25) (layer "B.Cu") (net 14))
 (segment (start 90.92 133) (end 99.08 133) (width 0.25) (layer "B.Cu") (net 14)))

